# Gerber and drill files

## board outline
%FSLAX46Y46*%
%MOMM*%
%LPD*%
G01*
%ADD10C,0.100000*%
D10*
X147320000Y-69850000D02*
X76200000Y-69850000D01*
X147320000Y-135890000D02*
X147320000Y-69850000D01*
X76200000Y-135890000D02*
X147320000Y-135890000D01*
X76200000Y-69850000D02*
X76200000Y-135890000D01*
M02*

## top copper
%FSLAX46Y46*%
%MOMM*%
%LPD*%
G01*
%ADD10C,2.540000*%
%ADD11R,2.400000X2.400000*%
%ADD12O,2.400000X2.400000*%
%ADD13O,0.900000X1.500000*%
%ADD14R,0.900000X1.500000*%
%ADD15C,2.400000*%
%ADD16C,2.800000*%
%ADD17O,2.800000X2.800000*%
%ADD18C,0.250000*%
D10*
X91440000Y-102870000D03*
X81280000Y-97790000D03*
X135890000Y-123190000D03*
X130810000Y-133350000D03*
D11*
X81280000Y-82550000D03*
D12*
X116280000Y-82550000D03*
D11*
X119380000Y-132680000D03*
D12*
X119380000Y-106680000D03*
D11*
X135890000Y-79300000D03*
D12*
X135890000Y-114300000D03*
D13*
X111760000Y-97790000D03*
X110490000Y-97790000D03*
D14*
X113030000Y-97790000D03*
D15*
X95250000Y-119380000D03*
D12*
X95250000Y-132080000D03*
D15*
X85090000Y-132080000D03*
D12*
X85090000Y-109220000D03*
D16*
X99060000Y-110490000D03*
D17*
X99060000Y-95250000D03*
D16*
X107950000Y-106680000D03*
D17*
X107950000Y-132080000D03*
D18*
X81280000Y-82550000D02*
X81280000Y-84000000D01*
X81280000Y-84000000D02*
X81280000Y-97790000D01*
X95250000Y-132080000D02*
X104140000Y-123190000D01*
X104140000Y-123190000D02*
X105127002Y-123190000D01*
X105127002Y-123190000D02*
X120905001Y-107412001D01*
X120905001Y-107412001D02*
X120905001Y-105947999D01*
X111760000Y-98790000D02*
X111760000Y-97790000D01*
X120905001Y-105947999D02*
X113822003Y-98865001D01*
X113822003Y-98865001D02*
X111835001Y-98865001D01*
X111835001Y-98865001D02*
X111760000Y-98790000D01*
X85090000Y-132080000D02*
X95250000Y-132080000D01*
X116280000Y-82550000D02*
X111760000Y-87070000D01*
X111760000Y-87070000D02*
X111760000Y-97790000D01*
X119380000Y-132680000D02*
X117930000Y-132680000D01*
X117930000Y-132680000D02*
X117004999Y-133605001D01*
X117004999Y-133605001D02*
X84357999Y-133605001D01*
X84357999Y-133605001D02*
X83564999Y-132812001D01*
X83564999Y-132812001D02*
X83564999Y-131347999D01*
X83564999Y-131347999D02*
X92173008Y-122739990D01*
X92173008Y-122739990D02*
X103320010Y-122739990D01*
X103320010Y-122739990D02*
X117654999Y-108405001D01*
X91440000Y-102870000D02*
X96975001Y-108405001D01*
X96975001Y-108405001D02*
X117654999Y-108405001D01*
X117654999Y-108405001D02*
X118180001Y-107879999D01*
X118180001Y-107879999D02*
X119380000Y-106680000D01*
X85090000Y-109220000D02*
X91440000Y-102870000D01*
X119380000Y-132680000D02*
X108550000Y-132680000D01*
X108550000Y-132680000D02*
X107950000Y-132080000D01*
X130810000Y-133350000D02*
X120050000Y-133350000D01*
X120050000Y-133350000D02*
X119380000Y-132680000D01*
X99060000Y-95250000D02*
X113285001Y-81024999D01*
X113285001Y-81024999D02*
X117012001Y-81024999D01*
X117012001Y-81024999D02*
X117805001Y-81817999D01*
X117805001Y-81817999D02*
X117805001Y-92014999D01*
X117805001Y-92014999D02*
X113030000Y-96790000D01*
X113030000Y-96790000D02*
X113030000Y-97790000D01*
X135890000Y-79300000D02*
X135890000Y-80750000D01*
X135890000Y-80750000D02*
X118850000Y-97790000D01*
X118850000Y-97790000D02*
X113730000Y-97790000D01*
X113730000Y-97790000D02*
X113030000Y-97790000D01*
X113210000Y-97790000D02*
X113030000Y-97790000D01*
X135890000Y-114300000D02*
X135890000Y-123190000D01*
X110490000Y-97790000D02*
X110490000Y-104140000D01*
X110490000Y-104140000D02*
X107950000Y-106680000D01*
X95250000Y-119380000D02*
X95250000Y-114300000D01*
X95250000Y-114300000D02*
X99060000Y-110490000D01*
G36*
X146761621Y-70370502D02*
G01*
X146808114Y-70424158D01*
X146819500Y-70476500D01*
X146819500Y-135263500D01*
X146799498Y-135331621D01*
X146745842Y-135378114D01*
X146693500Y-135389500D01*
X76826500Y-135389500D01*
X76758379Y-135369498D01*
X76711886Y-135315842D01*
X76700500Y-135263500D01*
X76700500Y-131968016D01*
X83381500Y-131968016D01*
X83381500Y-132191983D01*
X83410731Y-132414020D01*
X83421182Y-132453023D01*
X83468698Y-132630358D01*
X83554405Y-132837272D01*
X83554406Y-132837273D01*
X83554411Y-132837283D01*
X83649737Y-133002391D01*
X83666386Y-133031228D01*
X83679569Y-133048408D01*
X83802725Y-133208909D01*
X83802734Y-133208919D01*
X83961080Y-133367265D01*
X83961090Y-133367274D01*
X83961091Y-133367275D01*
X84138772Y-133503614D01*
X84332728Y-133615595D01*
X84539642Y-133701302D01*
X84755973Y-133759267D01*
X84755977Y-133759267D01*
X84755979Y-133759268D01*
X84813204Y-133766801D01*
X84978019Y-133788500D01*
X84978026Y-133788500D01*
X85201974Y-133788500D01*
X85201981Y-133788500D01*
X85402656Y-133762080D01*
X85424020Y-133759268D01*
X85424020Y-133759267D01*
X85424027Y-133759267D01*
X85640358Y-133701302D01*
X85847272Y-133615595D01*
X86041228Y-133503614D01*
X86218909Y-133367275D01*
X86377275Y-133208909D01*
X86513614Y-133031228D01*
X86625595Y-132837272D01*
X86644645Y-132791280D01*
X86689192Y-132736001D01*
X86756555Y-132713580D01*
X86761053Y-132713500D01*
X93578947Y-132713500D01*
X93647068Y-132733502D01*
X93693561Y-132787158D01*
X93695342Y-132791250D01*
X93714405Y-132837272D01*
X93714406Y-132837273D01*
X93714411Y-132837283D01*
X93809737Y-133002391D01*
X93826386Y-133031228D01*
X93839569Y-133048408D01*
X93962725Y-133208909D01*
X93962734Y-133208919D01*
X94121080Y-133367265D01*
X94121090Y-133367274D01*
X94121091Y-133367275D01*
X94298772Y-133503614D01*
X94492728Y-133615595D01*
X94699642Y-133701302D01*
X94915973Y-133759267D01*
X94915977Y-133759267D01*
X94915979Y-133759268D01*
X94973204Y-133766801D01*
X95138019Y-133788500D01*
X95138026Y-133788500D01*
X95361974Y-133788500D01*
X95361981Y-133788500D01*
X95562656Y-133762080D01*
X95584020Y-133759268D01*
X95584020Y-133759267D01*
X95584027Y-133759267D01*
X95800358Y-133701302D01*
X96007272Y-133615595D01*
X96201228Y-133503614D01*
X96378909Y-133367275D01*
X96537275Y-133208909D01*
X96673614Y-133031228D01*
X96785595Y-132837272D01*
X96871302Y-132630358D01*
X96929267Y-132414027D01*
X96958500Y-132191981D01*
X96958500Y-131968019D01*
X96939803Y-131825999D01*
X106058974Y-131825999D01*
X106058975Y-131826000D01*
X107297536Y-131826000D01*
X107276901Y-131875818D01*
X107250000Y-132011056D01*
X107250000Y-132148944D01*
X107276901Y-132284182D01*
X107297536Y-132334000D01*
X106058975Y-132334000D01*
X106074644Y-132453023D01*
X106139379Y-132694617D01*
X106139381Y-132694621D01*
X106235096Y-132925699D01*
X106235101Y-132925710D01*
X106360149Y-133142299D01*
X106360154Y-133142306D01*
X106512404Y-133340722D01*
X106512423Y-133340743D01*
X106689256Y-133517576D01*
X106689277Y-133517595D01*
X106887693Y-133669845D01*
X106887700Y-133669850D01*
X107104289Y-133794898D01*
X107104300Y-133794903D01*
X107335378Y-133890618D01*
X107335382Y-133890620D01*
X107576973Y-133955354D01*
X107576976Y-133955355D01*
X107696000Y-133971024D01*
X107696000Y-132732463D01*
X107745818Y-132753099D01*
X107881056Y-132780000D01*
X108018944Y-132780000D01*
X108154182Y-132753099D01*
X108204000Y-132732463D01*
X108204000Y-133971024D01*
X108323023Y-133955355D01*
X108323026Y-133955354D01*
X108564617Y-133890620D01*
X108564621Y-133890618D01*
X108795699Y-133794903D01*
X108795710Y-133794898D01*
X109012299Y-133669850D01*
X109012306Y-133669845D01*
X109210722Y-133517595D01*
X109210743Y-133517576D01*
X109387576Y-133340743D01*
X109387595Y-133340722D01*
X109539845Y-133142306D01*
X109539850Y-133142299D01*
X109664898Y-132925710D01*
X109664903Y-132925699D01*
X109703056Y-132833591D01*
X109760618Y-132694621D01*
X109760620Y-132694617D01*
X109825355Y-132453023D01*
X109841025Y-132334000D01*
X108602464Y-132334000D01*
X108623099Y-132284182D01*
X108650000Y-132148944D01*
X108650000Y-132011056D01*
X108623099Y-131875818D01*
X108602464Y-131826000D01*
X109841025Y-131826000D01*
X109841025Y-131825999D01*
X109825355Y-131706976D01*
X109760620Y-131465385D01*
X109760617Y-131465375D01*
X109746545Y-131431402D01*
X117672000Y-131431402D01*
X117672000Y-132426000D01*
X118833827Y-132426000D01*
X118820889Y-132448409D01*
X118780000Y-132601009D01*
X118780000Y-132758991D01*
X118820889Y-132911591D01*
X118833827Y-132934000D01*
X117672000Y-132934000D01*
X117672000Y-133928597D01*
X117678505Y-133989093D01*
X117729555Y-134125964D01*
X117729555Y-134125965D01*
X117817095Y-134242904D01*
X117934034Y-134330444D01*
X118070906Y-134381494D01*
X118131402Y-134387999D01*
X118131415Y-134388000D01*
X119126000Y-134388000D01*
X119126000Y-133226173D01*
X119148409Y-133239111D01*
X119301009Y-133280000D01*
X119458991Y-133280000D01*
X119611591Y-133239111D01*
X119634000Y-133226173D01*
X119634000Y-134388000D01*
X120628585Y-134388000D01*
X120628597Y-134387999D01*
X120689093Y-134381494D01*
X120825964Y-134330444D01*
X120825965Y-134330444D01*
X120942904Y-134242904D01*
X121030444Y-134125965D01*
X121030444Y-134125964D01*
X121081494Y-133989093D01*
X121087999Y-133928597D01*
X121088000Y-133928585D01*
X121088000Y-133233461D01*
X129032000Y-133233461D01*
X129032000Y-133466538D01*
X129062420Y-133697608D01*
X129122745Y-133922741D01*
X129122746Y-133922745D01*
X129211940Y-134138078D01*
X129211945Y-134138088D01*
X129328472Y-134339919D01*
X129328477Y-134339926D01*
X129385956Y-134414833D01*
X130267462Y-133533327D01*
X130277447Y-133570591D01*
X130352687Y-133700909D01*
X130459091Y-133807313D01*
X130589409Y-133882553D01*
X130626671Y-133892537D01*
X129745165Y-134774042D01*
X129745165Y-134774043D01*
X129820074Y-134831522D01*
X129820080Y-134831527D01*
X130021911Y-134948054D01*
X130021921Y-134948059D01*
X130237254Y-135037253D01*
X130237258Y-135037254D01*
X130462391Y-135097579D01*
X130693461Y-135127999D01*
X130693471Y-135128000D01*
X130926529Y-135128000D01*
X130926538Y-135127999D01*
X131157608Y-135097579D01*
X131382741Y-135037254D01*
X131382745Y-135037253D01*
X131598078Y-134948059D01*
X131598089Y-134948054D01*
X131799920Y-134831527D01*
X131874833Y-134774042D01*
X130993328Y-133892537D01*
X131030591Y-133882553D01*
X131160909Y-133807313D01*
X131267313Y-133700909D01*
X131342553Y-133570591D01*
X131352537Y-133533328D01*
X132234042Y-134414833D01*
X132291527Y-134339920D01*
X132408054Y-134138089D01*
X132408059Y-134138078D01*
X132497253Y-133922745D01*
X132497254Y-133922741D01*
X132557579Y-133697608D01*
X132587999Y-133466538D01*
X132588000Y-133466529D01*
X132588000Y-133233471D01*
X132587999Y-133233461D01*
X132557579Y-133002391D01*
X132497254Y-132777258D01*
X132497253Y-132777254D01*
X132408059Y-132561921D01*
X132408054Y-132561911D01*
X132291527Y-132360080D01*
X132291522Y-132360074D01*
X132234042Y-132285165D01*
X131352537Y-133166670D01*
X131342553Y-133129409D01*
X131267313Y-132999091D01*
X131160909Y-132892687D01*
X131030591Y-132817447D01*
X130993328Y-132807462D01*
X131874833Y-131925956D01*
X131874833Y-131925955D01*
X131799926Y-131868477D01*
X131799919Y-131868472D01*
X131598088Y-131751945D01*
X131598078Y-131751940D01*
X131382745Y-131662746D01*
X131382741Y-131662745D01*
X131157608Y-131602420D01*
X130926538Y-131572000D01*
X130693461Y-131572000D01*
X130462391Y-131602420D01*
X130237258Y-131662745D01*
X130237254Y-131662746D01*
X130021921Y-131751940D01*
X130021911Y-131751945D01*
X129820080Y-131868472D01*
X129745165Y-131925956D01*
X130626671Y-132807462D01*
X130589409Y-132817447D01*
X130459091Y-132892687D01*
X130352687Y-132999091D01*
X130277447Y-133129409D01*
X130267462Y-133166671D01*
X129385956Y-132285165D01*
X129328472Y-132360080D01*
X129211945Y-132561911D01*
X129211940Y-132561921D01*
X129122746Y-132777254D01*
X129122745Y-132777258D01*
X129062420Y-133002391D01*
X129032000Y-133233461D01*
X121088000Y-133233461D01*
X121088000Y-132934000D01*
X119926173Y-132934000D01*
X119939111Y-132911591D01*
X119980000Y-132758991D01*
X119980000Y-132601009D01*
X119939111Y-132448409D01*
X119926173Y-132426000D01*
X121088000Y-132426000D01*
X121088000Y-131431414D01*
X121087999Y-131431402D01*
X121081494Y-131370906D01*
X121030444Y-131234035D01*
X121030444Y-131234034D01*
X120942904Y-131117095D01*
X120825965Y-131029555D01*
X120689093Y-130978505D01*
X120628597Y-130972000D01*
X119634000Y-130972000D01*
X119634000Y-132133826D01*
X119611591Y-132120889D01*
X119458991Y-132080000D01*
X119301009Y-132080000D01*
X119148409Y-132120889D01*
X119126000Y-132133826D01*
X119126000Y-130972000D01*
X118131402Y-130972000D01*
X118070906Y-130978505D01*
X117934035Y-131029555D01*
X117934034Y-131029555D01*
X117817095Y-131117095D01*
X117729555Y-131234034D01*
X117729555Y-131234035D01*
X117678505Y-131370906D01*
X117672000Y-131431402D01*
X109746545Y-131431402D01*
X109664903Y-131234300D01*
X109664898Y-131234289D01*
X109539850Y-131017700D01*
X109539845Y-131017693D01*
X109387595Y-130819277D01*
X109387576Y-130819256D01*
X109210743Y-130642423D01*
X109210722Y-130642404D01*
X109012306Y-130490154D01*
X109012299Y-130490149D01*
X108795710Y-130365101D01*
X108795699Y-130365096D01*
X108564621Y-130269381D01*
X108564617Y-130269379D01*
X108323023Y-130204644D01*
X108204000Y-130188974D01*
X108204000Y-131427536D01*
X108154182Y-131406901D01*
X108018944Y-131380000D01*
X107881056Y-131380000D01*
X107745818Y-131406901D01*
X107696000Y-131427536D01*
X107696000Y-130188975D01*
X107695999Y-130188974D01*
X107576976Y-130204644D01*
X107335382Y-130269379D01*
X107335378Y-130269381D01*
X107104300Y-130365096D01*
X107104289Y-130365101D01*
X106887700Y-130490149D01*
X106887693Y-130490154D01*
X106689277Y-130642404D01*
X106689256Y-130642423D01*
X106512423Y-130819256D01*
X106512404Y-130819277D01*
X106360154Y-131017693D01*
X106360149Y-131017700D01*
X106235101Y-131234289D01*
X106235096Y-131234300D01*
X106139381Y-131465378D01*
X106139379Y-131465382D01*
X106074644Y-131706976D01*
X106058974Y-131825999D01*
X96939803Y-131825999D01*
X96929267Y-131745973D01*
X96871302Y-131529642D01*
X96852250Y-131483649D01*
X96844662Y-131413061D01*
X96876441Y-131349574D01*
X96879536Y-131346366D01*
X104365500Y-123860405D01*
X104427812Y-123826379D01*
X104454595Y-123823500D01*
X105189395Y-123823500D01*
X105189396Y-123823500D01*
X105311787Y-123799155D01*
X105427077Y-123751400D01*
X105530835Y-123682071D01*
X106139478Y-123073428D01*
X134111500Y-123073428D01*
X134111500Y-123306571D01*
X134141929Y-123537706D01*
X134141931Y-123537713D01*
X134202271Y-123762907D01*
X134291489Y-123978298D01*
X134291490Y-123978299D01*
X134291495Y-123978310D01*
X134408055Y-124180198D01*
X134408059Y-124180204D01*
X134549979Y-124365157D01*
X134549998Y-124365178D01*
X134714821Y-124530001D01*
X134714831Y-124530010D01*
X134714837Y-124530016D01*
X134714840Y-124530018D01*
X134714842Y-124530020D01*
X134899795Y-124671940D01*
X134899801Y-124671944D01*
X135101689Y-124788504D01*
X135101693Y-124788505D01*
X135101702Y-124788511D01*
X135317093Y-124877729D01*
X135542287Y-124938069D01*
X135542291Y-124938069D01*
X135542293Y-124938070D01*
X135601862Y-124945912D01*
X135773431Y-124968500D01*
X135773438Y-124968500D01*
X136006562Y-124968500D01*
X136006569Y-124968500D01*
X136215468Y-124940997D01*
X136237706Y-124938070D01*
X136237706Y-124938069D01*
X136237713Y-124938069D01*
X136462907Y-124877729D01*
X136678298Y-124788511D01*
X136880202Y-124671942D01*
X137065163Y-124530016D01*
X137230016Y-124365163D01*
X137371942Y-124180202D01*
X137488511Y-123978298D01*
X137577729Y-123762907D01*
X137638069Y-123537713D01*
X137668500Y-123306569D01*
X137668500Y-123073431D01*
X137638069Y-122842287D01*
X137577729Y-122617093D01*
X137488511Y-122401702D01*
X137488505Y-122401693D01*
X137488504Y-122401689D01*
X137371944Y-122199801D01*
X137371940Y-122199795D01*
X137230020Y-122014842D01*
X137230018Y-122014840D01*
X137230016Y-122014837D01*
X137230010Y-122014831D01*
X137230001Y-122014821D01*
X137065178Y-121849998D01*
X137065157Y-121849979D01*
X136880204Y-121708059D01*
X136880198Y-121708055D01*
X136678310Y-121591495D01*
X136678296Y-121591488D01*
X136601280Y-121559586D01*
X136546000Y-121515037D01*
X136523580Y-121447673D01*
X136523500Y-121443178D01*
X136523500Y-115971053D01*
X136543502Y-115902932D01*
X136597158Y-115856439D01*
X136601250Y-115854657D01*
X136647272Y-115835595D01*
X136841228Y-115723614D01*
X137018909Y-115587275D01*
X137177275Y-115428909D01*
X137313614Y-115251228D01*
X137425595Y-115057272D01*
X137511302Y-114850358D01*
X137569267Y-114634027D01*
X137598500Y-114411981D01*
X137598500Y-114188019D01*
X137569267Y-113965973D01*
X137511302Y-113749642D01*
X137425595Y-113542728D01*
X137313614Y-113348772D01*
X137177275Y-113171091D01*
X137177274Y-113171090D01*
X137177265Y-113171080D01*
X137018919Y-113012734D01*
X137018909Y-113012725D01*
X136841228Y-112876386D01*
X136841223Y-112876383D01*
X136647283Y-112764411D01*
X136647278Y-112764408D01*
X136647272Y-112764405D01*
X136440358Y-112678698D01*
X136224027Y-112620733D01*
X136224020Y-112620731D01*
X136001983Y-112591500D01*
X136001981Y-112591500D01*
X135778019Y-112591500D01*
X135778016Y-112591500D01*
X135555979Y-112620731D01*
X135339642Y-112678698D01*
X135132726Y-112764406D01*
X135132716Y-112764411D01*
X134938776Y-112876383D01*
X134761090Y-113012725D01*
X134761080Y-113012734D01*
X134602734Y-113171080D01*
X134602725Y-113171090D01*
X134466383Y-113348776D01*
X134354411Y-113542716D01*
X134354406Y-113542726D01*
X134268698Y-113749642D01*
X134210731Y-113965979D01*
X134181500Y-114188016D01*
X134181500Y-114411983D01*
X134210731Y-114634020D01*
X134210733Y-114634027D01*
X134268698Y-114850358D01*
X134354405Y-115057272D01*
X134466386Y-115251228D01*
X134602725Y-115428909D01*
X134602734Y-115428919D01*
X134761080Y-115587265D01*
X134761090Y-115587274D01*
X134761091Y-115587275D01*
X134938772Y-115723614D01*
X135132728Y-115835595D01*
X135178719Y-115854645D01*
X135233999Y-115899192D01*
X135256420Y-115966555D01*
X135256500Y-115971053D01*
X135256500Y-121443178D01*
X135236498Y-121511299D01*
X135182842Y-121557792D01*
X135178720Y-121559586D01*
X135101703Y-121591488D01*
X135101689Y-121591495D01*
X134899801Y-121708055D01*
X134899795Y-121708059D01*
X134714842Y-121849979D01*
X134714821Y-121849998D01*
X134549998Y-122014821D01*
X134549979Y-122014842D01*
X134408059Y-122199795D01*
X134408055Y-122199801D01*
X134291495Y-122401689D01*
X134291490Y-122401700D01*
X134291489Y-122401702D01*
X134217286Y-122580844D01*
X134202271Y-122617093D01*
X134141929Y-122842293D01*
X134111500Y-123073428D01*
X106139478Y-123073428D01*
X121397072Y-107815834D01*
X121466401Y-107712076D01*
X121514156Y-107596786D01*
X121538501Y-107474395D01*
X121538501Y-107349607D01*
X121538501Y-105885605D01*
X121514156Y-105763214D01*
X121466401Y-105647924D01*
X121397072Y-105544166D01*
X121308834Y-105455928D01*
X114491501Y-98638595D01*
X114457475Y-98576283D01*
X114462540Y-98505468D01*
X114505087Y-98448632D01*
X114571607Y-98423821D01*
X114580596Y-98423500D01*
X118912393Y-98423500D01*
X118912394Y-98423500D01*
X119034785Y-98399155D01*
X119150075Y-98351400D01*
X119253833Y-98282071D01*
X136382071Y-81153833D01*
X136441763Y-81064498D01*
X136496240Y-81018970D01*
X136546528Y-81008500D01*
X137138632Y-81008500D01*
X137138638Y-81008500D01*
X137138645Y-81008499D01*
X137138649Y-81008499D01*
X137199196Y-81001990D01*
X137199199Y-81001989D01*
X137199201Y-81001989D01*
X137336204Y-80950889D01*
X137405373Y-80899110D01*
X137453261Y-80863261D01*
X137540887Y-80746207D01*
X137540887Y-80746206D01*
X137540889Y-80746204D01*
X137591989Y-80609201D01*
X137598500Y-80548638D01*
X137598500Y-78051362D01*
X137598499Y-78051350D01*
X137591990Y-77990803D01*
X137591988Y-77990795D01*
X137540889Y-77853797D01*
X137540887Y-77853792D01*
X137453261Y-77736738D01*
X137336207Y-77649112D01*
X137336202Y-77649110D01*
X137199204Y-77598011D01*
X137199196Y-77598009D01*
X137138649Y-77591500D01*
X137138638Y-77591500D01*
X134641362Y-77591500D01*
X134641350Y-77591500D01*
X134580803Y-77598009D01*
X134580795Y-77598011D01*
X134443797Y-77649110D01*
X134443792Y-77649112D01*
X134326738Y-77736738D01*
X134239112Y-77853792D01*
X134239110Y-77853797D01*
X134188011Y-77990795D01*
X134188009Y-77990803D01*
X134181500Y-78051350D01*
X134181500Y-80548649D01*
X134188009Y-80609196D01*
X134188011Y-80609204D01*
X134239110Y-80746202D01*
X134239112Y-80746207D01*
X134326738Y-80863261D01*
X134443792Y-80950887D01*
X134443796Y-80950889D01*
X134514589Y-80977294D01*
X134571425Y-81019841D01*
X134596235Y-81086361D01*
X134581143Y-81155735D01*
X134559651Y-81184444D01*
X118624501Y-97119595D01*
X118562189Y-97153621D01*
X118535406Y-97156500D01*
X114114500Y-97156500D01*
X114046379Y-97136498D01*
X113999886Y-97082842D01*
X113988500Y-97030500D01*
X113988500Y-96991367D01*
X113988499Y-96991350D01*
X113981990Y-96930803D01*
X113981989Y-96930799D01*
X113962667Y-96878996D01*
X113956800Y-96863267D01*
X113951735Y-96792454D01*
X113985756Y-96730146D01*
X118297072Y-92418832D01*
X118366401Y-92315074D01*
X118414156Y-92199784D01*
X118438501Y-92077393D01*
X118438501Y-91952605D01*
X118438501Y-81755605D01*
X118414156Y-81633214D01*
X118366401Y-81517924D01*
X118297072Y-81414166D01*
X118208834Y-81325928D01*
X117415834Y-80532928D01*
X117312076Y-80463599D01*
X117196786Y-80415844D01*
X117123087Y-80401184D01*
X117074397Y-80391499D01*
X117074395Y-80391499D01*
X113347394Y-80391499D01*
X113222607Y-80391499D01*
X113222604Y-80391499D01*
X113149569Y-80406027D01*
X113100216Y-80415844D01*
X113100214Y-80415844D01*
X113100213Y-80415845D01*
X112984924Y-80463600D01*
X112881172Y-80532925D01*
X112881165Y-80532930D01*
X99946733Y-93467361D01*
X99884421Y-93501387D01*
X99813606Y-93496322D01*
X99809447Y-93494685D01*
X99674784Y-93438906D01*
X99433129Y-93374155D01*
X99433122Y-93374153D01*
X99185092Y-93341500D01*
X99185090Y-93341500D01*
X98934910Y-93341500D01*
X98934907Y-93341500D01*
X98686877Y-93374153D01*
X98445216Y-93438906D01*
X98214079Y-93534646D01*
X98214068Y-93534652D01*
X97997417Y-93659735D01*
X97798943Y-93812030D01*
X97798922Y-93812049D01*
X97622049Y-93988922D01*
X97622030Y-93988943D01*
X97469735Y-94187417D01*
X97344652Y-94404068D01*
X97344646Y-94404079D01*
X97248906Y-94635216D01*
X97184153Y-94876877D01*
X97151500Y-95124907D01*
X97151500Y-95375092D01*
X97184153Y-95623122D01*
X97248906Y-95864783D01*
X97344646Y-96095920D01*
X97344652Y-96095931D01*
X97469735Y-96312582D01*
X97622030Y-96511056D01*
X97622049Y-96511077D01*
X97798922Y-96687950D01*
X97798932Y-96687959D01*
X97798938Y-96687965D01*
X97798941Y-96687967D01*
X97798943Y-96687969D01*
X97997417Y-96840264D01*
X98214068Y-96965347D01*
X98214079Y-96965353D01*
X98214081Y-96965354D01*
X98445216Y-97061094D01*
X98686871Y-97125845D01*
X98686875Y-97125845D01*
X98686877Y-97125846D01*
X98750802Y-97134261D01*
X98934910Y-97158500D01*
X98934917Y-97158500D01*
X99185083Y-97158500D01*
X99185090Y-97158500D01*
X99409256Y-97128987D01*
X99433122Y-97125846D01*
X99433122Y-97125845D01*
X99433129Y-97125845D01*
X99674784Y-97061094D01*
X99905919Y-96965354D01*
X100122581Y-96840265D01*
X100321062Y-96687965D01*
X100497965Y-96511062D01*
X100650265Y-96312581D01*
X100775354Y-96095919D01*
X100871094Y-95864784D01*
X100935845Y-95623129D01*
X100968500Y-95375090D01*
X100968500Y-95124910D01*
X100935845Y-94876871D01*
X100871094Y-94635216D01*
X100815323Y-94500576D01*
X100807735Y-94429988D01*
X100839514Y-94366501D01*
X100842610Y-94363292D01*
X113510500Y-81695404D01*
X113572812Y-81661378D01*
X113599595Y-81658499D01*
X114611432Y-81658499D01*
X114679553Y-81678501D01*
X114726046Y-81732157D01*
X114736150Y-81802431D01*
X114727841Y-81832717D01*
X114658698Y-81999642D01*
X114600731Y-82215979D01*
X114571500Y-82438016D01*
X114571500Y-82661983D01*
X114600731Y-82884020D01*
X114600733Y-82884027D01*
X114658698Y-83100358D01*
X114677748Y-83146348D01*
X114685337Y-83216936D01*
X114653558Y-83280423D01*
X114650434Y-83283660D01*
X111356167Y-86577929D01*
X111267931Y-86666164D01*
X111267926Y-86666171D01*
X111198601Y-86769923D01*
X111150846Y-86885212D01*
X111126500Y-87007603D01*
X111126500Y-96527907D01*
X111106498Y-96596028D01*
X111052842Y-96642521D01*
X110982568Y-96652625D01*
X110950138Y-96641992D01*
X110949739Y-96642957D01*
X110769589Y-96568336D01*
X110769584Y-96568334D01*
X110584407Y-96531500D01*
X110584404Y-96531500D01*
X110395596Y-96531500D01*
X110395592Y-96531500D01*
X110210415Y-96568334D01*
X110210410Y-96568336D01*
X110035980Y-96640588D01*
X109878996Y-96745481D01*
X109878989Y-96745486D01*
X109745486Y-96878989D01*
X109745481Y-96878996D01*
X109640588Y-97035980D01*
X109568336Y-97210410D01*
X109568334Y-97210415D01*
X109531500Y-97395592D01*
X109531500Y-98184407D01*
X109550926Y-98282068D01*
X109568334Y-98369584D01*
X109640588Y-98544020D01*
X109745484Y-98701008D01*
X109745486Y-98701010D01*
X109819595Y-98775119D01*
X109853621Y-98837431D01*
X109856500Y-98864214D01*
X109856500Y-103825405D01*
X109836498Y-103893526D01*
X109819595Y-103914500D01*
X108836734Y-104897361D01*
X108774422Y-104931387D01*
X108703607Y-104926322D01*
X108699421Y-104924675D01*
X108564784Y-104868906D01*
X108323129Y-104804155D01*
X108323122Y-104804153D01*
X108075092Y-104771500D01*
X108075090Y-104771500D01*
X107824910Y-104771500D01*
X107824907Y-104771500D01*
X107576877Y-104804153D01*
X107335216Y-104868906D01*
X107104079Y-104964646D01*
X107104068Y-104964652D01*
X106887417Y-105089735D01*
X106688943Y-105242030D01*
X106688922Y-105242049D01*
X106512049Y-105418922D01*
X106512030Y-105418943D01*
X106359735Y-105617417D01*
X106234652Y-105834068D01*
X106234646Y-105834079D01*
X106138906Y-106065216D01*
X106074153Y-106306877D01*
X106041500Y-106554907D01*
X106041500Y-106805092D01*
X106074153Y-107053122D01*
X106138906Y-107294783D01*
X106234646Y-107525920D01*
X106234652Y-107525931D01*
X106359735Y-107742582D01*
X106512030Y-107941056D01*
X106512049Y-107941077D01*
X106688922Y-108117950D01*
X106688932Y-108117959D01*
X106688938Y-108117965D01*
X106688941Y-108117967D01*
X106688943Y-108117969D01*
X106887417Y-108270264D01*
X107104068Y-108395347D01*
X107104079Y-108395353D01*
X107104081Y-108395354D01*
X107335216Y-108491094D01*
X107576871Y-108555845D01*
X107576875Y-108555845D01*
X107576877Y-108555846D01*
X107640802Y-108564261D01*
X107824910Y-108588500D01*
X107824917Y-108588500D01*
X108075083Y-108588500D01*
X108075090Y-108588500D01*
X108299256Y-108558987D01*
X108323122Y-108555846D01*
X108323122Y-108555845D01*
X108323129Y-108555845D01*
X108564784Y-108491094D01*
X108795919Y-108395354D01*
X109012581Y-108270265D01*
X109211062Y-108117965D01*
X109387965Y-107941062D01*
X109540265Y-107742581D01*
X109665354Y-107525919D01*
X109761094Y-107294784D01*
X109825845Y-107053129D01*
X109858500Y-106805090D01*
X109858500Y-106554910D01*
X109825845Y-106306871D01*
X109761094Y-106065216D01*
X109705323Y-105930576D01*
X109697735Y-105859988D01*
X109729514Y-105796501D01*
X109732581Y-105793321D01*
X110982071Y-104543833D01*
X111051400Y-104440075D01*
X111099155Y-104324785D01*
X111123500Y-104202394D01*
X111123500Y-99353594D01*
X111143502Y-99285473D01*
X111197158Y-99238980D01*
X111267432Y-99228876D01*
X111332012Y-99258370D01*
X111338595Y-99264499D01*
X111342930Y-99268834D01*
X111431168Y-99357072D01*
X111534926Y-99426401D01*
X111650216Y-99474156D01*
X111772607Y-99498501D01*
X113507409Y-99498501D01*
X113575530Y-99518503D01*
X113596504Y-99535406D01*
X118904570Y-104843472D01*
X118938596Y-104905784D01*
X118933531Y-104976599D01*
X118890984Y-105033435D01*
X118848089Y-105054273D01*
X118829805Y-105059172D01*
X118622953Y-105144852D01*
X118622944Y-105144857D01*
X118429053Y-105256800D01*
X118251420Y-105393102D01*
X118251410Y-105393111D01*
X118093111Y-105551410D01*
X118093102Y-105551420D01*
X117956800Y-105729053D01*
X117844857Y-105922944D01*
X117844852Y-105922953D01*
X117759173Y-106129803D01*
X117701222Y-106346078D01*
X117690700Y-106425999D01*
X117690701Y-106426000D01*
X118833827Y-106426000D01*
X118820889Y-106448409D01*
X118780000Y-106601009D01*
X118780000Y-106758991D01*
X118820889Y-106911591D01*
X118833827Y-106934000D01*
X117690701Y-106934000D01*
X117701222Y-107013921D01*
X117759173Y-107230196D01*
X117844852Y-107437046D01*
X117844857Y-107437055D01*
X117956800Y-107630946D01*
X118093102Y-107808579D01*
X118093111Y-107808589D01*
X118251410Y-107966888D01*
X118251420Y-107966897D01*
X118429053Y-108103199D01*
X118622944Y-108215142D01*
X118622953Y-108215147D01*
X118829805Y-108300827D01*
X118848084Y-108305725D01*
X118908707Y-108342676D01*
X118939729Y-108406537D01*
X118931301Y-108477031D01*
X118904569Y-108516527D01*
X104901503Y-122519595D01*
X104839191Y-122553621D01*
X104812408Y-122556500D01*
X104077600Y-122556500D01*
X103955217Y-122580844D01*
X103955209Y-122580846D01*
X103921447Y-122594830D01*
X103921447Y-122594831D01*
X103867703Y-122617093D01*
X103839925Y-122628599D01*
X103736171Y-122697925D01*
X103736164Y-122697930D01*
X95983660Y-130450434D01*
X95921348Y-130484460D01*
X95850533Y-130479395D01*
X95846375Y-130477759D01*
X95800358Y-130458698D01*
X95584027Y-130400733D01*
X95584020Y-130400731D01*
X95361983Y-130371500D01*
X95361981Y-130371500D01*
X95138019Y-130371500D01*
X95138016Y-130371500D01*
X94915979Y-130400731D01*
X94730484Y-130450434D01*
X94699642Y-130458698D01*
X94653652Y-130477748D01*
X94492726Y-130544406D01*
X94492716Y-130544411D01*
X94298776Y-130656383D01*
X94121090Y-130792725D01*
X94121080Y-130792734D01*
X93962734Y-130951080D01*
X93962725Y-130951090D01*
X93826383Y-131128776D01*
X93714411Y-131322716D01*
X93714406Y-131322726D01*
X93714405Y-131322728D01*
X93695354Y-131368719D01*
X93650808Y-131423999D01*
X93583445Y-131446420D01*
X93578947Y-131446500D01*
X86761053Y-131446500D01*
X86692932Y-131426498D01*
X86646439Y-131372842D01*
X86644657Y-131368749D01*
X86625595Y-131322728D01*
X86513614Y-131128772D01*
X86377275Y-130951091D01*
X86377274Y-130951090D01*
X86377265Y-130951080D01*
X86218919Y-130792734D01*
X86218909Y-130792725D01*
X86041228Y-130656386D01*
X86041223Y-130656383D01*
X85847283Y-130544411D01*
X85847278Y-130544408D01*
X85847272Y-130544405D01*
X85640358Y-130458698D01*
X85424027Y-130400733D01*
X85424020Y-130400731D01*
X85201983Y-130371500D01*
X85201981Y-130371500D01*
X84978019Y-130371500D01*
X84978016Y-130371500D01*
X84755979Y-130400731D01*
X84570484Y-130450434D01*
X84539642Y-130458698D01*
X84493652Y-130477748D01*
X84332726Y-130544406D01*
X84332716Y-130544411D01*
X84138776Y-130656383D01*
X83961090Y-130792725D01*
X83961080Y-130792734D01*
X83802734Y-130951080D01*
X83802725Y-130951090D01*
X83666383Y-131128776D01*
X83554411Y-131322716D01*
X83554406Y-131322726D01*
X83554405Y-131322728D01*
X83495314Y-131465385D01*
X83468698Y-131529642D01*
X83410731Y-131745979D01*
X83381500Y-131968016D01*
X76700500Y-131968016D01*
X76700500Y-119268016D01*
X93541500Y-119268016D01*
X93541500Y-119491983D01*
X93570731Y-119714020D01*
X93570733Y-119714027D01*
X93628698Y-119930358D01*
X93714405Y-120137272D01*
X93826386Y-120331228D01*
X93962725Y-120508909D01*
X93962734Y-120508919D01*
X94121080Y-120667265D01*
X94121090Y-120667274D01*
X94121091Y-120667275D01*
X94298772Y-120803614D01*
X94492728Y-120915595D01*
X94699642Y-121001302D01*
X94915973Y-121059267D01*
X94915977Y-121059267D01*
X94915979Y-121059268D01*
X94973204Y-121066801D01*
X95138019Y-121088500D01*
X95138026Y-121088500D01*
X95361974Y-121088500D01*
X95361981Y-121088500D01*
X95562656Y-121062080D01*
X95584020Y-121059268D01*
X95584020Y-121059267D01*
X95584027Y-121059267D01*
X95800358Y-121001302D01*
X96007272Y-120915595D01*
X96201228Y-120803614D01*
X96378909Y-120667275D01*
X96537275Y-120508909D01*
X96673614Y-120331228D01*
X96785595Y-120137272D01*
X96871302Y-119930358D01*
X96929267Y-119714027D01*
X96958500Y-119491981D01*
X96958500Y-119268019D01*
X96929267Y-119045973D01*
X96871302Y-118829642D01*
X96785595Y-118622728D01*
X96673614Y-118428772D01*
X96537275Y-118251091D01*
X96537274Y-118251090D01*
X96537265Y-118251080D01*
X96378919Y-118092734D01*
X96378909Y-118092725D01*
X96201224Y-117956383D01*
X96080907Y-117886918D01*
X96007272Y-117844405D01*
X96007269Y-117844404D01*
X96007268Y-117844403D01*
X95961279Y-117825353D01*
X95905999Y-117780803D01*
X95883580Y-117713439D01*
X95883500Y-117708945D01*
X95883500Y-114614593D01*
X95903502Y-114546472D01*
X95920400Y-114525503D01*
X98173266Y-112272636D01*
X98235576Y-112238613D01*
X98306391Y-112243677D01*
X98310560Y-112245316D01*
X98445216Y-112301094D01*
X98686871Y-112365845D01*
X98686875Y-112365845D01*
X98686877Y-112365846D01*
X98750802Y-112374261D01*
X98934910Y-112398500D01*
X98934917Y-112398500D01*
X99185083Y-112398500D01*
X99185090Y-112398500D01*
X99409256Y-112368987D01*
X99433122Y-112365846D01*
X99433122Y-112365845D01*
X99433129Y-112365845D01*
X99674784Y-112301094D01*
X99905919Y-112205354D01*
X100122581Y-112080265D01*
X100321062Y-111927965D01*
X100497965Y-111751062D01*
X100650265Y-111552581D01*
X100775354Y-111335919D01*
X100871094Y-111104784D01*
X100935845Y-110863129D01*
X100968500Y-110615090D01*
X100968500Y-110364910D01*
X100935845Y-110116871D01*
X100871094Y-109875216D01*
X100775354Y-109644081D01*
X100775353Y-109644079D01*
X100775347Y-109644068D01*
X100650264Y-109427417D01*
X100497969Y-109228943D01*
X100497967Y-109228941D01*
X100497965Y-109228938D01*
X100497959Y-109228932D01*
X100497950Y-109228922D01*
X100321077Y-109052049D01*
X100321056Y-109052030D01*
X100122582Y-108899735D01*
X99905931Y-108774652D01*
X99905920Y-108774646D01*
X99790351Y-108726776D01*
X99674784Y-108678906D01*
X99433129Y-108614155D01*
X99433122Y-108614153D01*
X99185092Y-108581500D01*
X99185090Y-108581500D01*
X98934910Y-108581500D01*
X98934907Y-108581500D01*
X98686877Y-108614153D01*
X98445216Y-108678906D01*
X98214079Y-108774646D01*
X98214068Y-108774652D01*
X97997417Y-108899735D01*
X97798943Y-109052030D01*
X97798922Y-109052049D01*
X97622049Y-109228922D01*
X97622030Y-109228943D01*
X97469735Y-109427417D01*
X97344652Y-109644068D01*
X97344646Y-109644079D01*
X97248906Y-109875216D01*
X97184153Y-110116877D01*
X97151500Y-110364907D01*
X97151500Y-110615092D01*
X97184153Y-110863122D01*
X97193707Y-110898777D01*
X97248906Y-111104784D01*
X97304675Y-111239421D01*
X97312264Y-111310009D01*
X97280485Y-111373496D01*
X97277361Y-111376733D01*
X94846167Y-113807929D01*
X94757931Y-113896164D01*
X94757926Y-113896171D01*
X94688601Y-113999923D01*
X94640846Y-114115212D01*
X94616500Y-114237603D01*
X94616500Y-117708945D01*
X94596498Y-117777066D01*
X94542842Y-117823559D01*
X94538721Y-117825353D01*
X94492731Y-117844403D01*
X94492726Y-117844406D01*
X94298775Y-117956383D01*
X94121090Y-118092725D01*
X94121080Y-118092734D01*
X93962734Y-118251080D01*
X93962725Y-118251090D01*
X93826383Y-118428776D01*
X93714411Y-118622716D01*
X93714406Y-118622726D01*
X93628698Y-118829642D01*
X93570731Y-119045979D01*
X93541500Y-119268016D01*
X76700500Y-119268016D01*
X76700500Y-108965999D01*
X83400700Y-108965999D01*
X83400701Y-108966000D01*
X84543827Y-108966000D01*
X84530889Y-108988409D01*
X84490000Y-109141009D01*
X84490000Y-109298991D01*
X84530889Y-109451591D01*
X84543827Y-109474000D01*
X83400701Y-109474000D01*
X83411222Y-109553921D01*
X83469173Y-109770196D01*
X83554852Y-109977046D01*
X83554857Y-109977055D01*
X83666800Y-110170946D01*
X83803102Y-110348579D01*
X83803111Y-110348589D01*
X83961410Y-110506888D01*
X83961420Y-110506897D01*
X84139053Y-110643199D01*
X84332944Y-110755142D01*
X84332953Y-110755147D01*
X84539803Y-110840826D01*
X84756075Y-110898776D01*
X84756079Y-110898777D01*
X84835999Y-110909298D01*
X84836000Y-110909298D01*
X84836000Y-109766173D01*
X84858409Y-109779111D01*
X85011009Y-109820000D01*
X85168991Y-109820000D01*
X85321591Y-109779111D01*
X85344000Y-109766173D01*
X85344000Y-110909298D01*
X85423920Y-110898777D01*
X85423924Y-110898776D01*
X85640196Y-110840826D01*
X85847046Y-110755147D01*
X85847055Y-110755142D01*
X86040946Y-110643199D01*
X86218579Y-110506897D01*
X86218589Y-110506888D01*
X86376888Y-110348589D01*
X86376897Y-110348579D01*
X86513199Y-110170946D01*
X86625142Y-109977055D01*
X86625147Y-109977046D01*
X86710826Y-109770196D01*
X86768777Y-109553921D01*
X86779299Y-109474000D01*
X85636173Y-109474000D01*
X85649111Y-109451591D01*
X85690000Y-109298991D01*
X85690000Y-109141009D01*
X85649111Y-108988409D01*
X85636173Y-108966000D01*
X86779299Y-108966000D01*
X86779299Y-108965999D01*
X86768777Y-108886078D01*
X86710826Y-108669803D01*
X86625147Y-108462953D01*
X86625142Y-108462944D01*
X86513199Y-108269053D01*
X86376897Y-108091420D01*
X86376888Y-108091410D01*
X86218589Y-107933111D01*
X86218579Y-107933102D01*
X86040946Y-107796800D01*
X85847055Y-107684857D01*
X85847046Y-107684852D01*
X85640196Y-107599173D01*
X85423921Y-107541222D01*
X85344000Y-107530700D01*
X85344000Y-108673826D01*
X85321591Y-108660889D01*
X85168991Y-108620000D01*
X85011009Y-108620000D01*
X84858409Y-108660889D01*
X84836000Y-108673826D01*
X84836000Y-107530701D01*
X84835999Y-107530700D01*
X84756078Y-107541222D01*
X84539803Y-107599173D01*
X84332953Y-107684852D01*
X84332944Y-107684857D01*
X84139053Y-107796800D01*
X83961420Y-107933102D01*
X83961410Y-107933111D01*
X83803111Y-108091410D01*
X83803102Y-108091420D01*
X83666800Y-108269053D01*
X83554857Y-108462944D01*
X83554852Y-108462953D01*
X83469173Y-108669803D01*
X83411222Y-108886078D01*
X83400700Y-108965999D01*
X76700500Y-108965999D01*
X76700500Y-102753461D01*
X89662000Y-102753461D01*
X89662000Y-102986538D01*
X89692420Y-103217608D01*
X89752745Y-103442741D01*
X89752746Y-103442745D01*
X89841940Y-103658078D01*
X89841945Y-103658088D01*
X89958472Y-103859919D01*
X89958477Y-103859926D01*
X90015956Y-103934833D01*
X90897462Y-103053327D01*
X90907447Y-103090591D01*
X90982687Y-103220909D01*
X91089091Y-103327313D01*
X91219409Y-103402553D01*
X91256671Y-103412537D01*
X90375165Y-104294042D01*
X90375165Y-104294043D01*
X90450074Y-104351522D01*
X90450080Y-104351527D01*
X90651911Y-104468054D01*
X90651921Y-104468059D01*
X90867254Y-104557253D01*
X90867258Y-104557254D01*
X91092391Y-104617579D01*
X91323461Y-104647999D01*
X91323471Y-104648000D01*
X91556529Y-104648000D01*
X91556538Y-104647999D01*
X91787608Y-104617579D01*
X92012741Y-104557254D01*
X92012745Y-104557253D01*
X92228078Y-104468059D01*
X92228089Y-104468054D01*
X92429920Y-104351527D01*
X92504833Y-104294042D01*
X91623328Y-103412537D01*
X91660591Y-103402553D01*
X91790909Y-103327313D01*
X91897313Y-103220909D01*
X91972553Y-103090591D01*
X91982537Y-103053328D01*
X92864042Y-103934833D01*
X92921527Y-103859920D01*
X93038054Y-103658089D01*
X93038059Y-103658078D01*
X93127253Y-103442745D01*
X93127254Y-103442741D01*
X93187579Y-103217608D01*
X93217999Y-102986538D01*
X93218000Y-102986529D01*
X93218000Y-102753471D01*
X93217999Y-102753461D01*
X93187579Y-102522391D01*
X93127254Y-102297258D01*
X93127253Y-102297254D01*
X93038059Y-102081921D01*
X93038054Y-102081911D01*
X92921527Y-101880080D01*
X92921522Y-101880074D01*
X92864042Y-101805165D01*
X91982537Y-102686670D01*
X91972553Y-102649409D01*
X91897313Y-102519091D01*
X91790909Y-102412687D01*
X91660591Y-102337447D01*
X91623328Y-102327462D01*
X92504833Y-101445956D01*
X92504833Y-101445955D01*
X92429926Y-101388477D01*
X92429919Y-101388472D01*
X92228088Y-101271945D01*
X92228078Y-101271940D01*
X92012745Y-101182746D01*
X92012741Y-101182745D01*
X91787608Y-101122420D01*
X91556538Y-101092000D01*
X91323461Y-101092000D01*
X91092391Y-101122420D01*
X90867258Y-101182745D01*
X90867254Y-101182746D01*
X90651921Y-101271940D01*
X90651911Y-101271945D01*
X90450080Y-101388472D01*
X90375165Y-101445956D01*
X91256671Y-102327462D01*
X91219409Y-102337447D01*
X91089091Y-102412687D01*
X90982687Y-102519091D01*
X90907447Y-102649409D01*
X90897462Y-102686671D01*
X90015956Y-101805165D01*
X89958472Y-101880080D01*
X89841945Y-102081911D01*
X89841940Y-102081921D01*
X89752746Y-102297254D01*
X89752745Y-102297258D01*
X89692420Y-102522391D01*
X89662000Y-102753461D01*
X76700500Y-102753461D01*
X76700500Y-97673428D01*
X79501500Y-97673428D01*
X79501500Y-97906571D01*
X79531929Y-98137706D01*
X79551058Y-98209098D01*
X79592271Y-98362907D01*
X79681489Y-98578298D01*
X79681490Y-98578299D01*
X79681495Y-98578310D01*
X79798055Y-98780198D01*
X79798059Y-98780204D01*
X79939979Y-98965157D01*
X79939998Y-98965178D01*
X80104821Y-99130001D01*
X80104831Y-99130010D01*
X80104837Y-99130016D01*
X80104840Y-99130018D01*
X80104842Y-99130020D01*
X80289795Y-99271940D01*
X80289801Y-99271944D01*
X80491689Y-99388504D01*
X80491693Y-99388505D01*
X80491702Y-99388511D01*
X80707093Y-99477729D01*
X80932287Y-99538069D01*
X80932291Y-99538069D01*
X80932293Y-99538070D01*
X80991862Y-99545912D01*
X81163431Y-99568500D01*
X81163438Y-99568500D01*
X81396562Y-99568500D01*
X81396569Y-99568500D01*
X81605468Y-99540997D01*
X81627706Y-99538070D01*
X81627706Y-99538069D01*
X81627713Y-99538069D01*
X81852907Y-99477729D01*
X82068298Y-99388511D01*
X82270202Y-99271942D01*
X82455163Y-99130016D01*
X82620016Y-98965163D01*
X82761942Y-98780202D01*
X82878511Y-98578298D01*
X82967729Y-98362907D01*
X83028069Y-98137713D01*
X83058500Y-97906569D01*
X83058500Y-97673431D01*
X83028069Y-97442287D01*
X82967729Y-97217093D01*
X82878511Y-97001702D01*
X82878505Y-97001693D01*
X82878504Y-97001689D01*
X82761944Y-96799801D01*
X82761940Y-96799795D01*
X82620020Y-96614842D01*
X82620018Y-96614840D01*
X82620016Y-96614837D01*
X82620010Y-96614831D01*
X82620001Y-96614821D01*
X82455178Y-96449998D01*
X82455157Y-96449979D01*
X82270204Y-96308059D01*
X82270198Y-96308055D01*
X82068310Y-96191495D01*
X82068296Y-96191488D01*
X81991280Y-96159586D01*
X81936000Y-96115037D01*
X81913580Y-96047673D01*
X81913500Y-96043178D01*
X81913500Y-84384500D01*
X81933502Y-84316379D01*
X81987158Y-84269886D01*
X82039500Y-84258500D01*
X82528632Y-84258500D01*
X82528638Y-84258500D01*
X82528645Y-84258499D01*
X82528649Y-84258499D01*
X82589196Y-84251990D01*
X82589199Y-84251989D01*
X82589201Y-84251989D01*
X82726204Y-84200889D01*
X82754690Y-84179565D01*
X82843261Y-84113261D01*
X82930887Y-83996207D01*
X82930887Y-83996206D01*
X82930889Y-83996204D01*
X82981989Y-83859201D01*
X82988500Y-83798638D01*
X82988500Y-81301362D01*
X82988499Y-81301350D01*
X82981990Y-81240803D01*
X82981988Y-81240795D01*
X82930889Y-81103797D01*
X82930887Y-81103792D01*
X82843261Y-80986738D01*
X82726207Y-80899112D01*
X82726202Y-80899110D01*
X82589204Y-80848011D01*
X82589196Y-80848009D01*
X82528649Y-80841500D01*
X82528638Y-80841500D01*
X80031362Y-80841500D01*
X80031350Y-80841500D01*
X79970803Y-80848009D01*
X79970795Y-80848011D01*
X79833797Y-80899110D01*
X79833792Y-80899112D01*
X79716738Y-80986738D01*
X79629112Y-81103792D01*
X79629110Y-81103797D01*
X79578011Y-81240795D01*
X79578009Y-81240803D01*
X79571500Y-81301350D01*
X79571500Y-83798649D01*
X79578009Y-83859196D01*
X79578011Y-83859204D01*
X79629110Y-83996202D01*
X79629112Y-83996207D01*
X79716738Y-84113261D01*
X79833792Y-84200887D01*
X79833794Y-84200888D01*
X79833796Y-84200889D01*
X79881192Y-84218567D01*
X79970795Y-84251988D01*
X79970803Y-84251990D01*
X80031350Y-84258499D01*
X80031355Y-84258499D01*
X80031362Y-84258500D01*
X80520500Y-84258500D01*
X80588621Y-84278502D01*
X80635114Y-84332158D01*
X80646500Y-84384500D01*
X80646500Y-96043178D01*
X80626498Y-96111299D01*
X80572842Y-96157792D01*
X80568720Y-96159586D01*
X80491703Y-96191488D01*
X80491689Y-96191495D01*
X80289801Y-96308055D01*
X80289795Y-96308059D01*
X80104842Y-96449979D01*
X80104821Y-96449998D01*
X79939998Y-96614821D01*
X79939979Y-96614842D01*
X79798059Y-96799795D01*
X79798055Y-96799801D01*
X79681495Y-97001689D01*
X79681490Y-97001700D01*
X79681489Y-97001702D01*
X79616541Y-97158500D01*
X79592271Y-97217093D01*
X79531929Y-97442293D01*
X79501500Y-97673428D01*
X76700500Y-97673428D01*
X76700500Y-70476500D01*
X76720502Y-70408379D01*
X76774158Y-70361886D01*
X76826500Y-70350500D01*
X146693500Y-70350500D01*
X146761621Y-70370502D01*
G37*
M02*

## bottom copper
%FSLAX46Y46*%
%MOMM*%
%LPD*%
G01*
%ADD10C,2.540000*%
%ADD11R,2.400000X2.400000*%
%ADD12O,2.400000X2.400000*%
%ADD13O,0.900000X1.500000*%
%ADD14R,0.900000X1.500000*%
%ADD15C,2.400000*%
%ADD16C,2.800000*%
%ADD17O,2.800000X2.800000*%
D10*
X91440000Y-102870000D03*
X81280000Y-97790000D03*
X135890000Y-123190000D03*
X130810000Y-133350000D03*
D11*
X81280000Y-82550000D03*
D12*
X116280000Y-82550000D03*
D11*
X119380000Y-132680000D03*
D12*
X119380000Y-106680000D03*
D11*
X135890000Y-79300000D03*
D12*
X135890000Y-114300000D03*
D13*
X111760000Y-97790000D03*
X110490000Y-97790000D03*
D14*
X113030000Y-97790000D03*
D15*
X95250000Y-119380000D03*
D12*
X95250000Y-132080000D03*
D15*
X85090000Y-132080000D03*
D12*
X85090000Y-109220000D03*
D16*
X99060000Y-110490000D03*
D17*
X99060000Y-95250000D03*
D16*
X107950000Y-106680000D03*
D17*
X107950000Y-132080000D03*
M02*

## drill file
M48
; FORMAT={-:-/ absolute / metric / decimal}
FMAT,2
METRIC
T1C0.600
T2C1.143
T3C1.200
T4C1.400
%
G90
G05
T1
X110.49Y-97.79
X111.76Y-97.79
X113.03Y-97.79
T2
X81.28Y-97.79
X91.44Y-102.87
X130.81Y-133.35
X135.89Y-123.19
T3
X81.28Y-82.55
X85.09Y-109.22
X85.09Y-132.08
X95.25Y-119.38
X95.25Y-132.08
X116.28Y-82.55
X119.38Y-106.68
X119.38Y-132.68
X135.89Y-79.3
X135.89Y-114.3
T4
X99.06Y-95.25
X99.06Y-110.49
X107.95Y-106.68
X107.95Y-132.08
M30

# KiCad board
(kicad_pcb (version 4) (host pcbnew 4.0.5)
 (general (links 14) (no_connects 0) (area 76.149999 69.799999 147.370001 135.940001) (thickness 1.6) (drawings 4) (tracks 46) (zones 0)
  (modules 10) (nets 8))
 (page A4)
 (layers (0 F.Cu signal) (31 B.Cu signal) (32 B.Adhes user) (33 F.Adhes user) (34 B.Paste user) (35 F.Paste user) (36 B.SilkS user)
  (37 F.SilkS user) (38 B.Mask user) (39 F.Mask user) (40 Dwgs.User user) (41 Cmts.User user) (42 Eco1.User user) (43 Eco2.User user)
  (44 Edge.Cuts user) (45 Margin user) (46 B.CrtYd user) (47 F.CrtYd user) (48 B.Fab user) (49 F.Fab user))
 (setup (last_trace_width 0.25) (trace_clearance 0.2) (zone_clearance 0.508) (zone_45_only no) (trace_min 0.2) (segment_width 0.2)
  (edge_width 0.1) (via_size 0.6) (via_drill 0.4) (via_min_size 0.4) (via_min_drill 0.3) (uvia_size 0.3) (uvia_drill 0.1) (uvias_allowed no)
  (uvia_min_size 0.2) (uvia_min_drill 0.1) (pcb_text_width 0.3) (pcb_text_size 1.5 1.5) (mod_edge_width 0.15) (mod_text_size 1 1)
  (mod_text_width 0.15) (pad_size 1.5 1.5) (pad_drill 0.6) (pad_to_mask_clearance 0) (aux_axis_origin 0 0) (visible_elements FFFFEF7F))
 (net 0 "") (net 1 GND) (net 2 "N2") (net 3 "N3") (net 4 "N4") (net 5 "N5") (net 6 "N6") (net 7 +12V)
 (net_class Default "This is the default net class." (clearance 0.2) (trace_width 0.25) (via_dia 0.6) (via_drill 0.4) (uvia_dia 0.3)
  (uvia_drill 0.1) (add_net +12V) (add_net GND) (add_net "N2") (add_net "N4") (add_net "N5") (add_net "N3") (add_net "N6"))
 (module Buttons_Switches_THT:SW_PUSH (layer F.Cu) (at 86.36 100.33 180)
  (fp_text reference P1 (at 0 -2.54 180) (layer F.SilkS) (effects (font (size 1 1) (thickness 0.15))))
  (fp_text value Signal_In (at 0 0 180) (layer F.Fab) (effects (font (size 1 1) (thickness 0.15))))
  (pad 1 thru_hole circle (at -5.08 -2.54 180) (size 2.54 2.54) (drill 1.143) (layers *.Cu *.Mask) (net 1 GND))
  (pad 2 thru_hole circle (at 5.08 2.54 180) (size 2.54 2.54) (drill 1.143) (layers *.Cu *.Mask) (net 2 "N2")))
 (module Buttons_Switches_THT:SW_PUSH (layer F.Cu) (at 133.35 128.27 270)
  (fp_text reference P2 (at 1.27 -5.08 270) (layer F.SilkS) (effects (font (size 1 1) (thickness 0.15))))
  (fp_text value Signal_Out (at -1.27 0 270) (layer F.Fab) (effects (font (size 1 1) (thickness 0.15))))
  (pad 1 thru_hole circle (at -5.08 -2.54 270) (size 2.54 2.54) (drill 1.143) (layers *.Cu *.Mask) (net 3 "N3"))
  (pad 2 thru_hole circle (at 5.08 2.54 270) (size 2.54 2.54) (drill 1.143) (layers *.Cu *.Mask) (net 1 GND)))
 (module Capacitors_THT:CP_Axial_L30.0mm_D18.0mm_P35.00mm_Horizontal (layer F.Cu) (at 81.28 82.55)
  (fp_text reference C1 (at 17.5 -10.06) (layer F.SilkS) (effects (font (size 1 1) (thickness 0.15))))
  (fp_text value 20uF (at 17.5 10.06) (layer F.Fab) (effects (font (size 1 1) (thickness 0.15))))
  (pad 1 thru_hole rect (at 0 0) (size 2.4 2.4) (drill 1.2) (layers *.Cu *.Mask) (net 2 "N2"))
  (pad 2 thru_hole oval (at 35 0) (size 2.4 2.4) (drill 1.2) (layers *.Cu *.Mask) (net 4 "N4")))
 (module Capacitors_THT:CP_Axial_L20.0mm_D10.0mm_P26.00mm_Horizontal (layer F.Cu) (at 119.38 132.68 90)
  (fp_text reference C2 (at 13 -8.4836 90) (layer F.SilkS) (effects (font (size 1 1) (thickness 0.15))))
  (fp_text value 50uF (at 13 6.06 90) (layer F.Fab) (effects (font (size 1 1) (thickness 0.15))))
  (pad 1 thru_hole rect (at 0 0 90) (size 2.4 2.4) (drill 1.2) (layers *.Cu *.Mask) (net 1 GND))
  (pad 2 thru_hole oval (at 26 0 90) (size 2.4 2.4) (drill 1.2) (layers *.Cu *.Mask) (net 1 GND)))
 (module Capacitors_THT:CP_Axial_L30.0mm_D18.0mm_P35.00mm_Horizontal (layer F.Cu) (at 135.89 79.3 270)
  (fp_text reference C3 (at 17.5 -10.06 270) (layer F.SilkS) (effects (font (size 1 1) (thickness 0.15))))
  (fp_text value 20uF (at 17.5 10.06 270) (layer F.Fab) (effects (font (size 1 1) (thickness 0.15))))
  (pad 1 thru_hole rect (at 0 0 270) (size 2.4 2.4) (drill 1.2) (layers *.Cu *.Mask) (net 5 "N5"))
  (pad 2 thru_hole oval (at 35 0 270) (size 2.4 2.4) (drill 1.2) (layers *.Cu *.Mask) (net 3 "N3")))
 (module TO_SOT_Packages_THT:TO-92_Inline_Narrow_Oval (layer F.Cu) (at 113.03 97.79 180)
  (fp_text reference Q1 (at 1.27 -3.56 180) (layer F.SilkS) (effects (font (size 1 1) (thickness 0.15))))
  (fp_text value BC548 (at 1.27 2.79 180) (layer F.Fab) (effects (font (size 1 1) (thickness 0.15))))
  (pad 2 thru_hole oval (at 1.27 0) (size 0.9 1.5) (drill 0.6) (layers *.Cu *.Mask) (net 4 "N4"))
  (pad 3 thru_hole oval (at 2.54 0) (size 0.9 1.5) (drill 0.6) (layers *.Cu *.Mask) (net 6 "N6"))
  (pad 1 thru_hole rect (at 0 0) (size 0.9 1.5) (drill 0.6) (layers *.Cu *.Mask) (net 5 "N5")))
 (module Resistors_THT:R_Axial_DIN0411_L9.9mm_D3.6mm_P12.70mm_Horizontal (layer F.Cu) (at 95.25 119.38 270)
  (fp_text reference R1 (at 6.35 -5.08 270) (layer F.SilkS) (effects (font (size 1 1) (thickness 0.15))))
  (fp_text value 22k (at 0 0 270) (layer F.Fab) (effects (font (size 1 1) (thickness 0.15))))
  (pad 1 thru_hole circle (at 0 0 270) (size 2.4 2.4) (drill 1.2) (layers *.Cu *.Mask) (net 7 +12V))
  (pad 2 thru_hole oval (at 12.7 0 270) (size 2.4 2.4) (drill 1.2) (layers *.Cu *.Mask) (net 4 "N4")))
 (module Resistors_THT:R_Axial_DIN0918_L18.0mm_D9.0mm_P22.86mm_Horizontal (layer F.Cu) (at 85.09 132.08 90)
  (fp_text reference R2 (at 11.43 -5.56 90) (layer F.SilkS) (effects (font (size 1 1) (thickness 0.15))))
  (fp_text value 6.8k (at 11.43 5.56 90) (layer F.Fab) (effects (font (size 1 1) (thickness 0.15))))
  (pad 1 thru_hole circle (at 0 0 90) (size 2.4 2.4) (drill 1.2) (layers *.Cu *.Mask) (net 4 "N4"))
  (pad 2 thru_hole oval (at 22.86 0 90) (size 2.4 2.4) (drill 1.2) (layers *.Cu *.Mask) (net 1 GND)))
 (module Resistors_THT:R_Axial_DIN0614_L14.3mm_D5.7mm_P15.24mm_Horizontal (layer F.Cu) (at 99.06 110.49 90)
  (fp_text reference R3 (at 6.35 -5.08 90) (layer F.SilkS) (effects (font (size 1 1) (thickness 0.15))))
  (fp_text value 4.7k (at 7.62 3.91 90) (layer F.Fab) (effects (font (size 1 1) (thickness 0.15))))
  (pad 1 thru_hole circle (at 0 0 90) (size 2.8 2.8) (drill 1.4) (layers *.Cu *.Mask) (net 7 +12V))
  (pad 2 thru_hole oval (at 15.24 0 90) (size 2.8 2.8) (drill 1.4) (layers *.Cu *.Mask) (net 5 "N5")))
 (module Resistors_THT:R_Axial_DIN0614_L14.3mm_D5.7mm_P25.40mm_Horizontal (layer F.Cu) (at 107.95 106.68 270)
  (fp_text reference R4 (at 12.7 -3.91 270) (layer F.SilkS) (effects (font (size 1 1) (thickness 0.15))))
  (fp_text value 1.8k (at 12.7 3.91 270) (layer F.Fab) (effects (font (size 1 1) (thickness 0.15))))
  (pad 1 thru_hole circle (at 0 0 270) (size 2.8 2.8) (drill 1.4) (layers *.Cu *.Mask) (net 6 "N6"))
  (pad 2 thru_hole oval (at 25.4 0 270) (size 2.8 2.8) (drill 1.4) (layers *.Cu *.Mask) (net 1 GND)))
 (gr_line (start 147.32 69.85) (end 76.2 69.85) (layer Edge.Cuts) (width 0.1))
 (gr_line (start 147.32 135.89) (end 147.32 69.85) (layer Edge.Cuts) (width 0.1))
 (gr_line (start 76.2 135.89) (end 147.32 135.89) (layer Edge.Cuts) (width 0.1))
 (gr_line (start 76.2 69.85) (end 76.2 135.89) (layer Edge.Cuts) (width 0.1))
 (segment (start 81.28 82.55) (end 81.28 84) (width 0.25) (layer F.Cu) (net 2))
 (segment (start 81.28 84) (end 81.28 97.79) (width 0.25) (layer F.Cu) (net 2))
 (segment (start 95.25 132.08) (end 104.14 123.19) (width 0.25) (layer F.Cu) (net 4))
 (segment (start 104.14 123.19) (end 105.127002 123.19) (width 0.25) (layer F.Cu) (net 4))
 (segment (start 105.127002 123.19) (end 120.905001 107.412001) (width 0.25) (layer F.Cu) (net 4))
 (segment (start 120.905001 107.412001) (end 120.905001 105.947999) (width 0.25) (layer F.Cu) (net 4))
 (segment (start 111.76 98.79) (end 111.76 97.79) (width 0.25) (layer F.Cu) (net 4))
 (segment (start 120.905001 105.947999) (end 113.822003 98.865001) (width 0.25) (layer F.Cu) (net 4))
 (segment (start 113.822003 98.865001) (end 111.835001 98.865001) (width 0.25) (layer F.Cu) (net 4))
 (segment (start 111.835001 98.865001) (end 111.76 98.79) (width 0.25) (layer F.Cu) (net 4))
 (segment (start 85.09 132.08) (end 95.25 132.08) (width 0.25) (layer F.Cu) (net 4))
 (segment (start 116.28 82.55) (end 111.76 87.07) (width 0.25) (layer F.Cu) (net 4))
 (segment (start 111.76 87.07) (end 111.76 97.79) (width 0.25) (layer F.Cu) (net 4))
 (segment (start 119.38 132.68) (end 117.93 132.68) (width 0.25) (layer F.Cu) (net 1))
 (segment (start 117.93 132.68) (end 117.004999 133.605001) (width 0.25) (layer F.Cu) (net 1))
 (segment (start 117.004999 133.605001) (end 84.357999 133.605001) (width 0.25) (layer F.Cu) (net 1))
 (segment (start 84.357999 133.605001) (end 83.564999 132.812001) (width 0.25) (layer F.Cu) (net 1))
 (segment (start 83.564999 132.812001) (end 83.564999 131.347999) (width 0.25) (layer F.Cu) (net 1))
 (segment (start 83.564999 131.347999) (end 92.173008 122.73999) (width 0.25) (layer F.Cu) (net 1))
 (segment (start 92.173008 122.73999) (end 103.32001 122.73999) (width 0.25) (layer F.Cu) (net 1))
 (segment (start 103.32001 122.73999) (end 117.654999 108.405001) (width 0.25) (layer F.Cu) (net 1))
 (segment (start 91.44 102.87) (end 96.975001 108.405001) (width 0.25) (layer F.Cu) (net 1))
 (segment (start 96.975001 108.405001) (end 117.654999 108.405001) (width 0.25) (layer F.Cu) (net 1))
 (segment (start 117.654999 108.405001) (end 118.180001 107.879999) (width 0.25) (layer F.Cu) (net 1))
 (segment (start 118.180001 107.879999) (end 119.38 106.68) (width 0.25) (layer F.Cu) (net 1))
 (segment (start 85.09 109.22) (end 91.44 102.87) (width 0.25) (layer F.Cu) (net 1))
 (segment (start 119.38 132.68) (end 108.55 132.68) (width 0.25) (layer F.Cu) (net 1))
 (segment (start 108.55 132.68) (end 107.95 132.08) (width 0.25) (layer F.Cu) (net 1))
 (segment (start 130.81 133.35) (end 120.05 133.35) (width 0.25) (layer F.Cu) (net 1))
 (segment (start 120.05 133.35) (end 119.38 132.68) (width 0.25) (layer F.Cu) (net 1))
 (segment (start 99.06 95.25) (end 113.285001 81.024999) (width 0.25) (layer F.Cu) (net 5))
 (segment (start 113.285001 81.024999) (end 117.012001 81.024999) (width 0.25) (layer F.Cu) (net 5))
 (segment (start 117.012001 81.024999) (end 117.805001 81.817999) (width 0.25) (layer F.Cu) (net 5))
 (segment (start 117.805001 81.817999) (end 117.805001 92.014999) (width 0.25) (layer F.Cu) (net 5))
 (segment (start 117.805001 92.014999) (end 113.03 96.79) (width 0.25) (layer F.Cu) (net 5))
 (segment (start 113.03 96.79) (end 113.03 97.79) (width 0.25) (layer F.Cu) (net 5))
 (segment (start 135.89 79.3) (end 135.89 80.75) (width 0.25) (layer F.Cu) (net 5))
 (segment (start 135.89 80.75) (end 118.85 97.79) (width 0.25) (layer F.Cu) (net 5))
 (segment (start 118.85 97.79) (end 113.73 97.79) (width 0.25) (layer F.Cu) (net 5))
 (segment (start 113.73 97.79) (end 113.03 97.79) (width 0.25) (layer F.Cu) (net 5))
 (segment (start 113.21 97.79) (end 113.03 97.79) (width 0.25) (layer F.Cu) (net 5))
 (segment (start 135.89 114.3) (end 135.89 123.19) (width 0.25) (layer F.Cu) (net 3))
 (segment (start 110.49 97.79) (end 110.49 104.14) (width 0.25) (layer F.Cu) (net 6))
 (segment (start 110.49 104.14) (end 107.95 106.68) (width 0.25) (layer F.Cu) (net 6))
 (segment (start 95.25 119.38) (end 95.25 114.3) (width 0.25) (layer F.Cu) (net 7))
 (segment (start 95.25 114.3) (end 99.06 110.49) (width 0.25) (layer F.Cu) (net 7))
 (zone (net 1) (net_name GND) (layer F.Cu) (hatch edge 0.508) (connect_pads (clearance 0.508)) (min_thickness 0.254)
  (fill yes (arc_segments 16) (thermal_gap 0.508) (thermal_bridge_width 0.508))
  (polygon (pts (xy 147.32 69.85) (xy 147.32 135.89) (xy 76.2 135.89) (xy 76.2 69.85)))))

